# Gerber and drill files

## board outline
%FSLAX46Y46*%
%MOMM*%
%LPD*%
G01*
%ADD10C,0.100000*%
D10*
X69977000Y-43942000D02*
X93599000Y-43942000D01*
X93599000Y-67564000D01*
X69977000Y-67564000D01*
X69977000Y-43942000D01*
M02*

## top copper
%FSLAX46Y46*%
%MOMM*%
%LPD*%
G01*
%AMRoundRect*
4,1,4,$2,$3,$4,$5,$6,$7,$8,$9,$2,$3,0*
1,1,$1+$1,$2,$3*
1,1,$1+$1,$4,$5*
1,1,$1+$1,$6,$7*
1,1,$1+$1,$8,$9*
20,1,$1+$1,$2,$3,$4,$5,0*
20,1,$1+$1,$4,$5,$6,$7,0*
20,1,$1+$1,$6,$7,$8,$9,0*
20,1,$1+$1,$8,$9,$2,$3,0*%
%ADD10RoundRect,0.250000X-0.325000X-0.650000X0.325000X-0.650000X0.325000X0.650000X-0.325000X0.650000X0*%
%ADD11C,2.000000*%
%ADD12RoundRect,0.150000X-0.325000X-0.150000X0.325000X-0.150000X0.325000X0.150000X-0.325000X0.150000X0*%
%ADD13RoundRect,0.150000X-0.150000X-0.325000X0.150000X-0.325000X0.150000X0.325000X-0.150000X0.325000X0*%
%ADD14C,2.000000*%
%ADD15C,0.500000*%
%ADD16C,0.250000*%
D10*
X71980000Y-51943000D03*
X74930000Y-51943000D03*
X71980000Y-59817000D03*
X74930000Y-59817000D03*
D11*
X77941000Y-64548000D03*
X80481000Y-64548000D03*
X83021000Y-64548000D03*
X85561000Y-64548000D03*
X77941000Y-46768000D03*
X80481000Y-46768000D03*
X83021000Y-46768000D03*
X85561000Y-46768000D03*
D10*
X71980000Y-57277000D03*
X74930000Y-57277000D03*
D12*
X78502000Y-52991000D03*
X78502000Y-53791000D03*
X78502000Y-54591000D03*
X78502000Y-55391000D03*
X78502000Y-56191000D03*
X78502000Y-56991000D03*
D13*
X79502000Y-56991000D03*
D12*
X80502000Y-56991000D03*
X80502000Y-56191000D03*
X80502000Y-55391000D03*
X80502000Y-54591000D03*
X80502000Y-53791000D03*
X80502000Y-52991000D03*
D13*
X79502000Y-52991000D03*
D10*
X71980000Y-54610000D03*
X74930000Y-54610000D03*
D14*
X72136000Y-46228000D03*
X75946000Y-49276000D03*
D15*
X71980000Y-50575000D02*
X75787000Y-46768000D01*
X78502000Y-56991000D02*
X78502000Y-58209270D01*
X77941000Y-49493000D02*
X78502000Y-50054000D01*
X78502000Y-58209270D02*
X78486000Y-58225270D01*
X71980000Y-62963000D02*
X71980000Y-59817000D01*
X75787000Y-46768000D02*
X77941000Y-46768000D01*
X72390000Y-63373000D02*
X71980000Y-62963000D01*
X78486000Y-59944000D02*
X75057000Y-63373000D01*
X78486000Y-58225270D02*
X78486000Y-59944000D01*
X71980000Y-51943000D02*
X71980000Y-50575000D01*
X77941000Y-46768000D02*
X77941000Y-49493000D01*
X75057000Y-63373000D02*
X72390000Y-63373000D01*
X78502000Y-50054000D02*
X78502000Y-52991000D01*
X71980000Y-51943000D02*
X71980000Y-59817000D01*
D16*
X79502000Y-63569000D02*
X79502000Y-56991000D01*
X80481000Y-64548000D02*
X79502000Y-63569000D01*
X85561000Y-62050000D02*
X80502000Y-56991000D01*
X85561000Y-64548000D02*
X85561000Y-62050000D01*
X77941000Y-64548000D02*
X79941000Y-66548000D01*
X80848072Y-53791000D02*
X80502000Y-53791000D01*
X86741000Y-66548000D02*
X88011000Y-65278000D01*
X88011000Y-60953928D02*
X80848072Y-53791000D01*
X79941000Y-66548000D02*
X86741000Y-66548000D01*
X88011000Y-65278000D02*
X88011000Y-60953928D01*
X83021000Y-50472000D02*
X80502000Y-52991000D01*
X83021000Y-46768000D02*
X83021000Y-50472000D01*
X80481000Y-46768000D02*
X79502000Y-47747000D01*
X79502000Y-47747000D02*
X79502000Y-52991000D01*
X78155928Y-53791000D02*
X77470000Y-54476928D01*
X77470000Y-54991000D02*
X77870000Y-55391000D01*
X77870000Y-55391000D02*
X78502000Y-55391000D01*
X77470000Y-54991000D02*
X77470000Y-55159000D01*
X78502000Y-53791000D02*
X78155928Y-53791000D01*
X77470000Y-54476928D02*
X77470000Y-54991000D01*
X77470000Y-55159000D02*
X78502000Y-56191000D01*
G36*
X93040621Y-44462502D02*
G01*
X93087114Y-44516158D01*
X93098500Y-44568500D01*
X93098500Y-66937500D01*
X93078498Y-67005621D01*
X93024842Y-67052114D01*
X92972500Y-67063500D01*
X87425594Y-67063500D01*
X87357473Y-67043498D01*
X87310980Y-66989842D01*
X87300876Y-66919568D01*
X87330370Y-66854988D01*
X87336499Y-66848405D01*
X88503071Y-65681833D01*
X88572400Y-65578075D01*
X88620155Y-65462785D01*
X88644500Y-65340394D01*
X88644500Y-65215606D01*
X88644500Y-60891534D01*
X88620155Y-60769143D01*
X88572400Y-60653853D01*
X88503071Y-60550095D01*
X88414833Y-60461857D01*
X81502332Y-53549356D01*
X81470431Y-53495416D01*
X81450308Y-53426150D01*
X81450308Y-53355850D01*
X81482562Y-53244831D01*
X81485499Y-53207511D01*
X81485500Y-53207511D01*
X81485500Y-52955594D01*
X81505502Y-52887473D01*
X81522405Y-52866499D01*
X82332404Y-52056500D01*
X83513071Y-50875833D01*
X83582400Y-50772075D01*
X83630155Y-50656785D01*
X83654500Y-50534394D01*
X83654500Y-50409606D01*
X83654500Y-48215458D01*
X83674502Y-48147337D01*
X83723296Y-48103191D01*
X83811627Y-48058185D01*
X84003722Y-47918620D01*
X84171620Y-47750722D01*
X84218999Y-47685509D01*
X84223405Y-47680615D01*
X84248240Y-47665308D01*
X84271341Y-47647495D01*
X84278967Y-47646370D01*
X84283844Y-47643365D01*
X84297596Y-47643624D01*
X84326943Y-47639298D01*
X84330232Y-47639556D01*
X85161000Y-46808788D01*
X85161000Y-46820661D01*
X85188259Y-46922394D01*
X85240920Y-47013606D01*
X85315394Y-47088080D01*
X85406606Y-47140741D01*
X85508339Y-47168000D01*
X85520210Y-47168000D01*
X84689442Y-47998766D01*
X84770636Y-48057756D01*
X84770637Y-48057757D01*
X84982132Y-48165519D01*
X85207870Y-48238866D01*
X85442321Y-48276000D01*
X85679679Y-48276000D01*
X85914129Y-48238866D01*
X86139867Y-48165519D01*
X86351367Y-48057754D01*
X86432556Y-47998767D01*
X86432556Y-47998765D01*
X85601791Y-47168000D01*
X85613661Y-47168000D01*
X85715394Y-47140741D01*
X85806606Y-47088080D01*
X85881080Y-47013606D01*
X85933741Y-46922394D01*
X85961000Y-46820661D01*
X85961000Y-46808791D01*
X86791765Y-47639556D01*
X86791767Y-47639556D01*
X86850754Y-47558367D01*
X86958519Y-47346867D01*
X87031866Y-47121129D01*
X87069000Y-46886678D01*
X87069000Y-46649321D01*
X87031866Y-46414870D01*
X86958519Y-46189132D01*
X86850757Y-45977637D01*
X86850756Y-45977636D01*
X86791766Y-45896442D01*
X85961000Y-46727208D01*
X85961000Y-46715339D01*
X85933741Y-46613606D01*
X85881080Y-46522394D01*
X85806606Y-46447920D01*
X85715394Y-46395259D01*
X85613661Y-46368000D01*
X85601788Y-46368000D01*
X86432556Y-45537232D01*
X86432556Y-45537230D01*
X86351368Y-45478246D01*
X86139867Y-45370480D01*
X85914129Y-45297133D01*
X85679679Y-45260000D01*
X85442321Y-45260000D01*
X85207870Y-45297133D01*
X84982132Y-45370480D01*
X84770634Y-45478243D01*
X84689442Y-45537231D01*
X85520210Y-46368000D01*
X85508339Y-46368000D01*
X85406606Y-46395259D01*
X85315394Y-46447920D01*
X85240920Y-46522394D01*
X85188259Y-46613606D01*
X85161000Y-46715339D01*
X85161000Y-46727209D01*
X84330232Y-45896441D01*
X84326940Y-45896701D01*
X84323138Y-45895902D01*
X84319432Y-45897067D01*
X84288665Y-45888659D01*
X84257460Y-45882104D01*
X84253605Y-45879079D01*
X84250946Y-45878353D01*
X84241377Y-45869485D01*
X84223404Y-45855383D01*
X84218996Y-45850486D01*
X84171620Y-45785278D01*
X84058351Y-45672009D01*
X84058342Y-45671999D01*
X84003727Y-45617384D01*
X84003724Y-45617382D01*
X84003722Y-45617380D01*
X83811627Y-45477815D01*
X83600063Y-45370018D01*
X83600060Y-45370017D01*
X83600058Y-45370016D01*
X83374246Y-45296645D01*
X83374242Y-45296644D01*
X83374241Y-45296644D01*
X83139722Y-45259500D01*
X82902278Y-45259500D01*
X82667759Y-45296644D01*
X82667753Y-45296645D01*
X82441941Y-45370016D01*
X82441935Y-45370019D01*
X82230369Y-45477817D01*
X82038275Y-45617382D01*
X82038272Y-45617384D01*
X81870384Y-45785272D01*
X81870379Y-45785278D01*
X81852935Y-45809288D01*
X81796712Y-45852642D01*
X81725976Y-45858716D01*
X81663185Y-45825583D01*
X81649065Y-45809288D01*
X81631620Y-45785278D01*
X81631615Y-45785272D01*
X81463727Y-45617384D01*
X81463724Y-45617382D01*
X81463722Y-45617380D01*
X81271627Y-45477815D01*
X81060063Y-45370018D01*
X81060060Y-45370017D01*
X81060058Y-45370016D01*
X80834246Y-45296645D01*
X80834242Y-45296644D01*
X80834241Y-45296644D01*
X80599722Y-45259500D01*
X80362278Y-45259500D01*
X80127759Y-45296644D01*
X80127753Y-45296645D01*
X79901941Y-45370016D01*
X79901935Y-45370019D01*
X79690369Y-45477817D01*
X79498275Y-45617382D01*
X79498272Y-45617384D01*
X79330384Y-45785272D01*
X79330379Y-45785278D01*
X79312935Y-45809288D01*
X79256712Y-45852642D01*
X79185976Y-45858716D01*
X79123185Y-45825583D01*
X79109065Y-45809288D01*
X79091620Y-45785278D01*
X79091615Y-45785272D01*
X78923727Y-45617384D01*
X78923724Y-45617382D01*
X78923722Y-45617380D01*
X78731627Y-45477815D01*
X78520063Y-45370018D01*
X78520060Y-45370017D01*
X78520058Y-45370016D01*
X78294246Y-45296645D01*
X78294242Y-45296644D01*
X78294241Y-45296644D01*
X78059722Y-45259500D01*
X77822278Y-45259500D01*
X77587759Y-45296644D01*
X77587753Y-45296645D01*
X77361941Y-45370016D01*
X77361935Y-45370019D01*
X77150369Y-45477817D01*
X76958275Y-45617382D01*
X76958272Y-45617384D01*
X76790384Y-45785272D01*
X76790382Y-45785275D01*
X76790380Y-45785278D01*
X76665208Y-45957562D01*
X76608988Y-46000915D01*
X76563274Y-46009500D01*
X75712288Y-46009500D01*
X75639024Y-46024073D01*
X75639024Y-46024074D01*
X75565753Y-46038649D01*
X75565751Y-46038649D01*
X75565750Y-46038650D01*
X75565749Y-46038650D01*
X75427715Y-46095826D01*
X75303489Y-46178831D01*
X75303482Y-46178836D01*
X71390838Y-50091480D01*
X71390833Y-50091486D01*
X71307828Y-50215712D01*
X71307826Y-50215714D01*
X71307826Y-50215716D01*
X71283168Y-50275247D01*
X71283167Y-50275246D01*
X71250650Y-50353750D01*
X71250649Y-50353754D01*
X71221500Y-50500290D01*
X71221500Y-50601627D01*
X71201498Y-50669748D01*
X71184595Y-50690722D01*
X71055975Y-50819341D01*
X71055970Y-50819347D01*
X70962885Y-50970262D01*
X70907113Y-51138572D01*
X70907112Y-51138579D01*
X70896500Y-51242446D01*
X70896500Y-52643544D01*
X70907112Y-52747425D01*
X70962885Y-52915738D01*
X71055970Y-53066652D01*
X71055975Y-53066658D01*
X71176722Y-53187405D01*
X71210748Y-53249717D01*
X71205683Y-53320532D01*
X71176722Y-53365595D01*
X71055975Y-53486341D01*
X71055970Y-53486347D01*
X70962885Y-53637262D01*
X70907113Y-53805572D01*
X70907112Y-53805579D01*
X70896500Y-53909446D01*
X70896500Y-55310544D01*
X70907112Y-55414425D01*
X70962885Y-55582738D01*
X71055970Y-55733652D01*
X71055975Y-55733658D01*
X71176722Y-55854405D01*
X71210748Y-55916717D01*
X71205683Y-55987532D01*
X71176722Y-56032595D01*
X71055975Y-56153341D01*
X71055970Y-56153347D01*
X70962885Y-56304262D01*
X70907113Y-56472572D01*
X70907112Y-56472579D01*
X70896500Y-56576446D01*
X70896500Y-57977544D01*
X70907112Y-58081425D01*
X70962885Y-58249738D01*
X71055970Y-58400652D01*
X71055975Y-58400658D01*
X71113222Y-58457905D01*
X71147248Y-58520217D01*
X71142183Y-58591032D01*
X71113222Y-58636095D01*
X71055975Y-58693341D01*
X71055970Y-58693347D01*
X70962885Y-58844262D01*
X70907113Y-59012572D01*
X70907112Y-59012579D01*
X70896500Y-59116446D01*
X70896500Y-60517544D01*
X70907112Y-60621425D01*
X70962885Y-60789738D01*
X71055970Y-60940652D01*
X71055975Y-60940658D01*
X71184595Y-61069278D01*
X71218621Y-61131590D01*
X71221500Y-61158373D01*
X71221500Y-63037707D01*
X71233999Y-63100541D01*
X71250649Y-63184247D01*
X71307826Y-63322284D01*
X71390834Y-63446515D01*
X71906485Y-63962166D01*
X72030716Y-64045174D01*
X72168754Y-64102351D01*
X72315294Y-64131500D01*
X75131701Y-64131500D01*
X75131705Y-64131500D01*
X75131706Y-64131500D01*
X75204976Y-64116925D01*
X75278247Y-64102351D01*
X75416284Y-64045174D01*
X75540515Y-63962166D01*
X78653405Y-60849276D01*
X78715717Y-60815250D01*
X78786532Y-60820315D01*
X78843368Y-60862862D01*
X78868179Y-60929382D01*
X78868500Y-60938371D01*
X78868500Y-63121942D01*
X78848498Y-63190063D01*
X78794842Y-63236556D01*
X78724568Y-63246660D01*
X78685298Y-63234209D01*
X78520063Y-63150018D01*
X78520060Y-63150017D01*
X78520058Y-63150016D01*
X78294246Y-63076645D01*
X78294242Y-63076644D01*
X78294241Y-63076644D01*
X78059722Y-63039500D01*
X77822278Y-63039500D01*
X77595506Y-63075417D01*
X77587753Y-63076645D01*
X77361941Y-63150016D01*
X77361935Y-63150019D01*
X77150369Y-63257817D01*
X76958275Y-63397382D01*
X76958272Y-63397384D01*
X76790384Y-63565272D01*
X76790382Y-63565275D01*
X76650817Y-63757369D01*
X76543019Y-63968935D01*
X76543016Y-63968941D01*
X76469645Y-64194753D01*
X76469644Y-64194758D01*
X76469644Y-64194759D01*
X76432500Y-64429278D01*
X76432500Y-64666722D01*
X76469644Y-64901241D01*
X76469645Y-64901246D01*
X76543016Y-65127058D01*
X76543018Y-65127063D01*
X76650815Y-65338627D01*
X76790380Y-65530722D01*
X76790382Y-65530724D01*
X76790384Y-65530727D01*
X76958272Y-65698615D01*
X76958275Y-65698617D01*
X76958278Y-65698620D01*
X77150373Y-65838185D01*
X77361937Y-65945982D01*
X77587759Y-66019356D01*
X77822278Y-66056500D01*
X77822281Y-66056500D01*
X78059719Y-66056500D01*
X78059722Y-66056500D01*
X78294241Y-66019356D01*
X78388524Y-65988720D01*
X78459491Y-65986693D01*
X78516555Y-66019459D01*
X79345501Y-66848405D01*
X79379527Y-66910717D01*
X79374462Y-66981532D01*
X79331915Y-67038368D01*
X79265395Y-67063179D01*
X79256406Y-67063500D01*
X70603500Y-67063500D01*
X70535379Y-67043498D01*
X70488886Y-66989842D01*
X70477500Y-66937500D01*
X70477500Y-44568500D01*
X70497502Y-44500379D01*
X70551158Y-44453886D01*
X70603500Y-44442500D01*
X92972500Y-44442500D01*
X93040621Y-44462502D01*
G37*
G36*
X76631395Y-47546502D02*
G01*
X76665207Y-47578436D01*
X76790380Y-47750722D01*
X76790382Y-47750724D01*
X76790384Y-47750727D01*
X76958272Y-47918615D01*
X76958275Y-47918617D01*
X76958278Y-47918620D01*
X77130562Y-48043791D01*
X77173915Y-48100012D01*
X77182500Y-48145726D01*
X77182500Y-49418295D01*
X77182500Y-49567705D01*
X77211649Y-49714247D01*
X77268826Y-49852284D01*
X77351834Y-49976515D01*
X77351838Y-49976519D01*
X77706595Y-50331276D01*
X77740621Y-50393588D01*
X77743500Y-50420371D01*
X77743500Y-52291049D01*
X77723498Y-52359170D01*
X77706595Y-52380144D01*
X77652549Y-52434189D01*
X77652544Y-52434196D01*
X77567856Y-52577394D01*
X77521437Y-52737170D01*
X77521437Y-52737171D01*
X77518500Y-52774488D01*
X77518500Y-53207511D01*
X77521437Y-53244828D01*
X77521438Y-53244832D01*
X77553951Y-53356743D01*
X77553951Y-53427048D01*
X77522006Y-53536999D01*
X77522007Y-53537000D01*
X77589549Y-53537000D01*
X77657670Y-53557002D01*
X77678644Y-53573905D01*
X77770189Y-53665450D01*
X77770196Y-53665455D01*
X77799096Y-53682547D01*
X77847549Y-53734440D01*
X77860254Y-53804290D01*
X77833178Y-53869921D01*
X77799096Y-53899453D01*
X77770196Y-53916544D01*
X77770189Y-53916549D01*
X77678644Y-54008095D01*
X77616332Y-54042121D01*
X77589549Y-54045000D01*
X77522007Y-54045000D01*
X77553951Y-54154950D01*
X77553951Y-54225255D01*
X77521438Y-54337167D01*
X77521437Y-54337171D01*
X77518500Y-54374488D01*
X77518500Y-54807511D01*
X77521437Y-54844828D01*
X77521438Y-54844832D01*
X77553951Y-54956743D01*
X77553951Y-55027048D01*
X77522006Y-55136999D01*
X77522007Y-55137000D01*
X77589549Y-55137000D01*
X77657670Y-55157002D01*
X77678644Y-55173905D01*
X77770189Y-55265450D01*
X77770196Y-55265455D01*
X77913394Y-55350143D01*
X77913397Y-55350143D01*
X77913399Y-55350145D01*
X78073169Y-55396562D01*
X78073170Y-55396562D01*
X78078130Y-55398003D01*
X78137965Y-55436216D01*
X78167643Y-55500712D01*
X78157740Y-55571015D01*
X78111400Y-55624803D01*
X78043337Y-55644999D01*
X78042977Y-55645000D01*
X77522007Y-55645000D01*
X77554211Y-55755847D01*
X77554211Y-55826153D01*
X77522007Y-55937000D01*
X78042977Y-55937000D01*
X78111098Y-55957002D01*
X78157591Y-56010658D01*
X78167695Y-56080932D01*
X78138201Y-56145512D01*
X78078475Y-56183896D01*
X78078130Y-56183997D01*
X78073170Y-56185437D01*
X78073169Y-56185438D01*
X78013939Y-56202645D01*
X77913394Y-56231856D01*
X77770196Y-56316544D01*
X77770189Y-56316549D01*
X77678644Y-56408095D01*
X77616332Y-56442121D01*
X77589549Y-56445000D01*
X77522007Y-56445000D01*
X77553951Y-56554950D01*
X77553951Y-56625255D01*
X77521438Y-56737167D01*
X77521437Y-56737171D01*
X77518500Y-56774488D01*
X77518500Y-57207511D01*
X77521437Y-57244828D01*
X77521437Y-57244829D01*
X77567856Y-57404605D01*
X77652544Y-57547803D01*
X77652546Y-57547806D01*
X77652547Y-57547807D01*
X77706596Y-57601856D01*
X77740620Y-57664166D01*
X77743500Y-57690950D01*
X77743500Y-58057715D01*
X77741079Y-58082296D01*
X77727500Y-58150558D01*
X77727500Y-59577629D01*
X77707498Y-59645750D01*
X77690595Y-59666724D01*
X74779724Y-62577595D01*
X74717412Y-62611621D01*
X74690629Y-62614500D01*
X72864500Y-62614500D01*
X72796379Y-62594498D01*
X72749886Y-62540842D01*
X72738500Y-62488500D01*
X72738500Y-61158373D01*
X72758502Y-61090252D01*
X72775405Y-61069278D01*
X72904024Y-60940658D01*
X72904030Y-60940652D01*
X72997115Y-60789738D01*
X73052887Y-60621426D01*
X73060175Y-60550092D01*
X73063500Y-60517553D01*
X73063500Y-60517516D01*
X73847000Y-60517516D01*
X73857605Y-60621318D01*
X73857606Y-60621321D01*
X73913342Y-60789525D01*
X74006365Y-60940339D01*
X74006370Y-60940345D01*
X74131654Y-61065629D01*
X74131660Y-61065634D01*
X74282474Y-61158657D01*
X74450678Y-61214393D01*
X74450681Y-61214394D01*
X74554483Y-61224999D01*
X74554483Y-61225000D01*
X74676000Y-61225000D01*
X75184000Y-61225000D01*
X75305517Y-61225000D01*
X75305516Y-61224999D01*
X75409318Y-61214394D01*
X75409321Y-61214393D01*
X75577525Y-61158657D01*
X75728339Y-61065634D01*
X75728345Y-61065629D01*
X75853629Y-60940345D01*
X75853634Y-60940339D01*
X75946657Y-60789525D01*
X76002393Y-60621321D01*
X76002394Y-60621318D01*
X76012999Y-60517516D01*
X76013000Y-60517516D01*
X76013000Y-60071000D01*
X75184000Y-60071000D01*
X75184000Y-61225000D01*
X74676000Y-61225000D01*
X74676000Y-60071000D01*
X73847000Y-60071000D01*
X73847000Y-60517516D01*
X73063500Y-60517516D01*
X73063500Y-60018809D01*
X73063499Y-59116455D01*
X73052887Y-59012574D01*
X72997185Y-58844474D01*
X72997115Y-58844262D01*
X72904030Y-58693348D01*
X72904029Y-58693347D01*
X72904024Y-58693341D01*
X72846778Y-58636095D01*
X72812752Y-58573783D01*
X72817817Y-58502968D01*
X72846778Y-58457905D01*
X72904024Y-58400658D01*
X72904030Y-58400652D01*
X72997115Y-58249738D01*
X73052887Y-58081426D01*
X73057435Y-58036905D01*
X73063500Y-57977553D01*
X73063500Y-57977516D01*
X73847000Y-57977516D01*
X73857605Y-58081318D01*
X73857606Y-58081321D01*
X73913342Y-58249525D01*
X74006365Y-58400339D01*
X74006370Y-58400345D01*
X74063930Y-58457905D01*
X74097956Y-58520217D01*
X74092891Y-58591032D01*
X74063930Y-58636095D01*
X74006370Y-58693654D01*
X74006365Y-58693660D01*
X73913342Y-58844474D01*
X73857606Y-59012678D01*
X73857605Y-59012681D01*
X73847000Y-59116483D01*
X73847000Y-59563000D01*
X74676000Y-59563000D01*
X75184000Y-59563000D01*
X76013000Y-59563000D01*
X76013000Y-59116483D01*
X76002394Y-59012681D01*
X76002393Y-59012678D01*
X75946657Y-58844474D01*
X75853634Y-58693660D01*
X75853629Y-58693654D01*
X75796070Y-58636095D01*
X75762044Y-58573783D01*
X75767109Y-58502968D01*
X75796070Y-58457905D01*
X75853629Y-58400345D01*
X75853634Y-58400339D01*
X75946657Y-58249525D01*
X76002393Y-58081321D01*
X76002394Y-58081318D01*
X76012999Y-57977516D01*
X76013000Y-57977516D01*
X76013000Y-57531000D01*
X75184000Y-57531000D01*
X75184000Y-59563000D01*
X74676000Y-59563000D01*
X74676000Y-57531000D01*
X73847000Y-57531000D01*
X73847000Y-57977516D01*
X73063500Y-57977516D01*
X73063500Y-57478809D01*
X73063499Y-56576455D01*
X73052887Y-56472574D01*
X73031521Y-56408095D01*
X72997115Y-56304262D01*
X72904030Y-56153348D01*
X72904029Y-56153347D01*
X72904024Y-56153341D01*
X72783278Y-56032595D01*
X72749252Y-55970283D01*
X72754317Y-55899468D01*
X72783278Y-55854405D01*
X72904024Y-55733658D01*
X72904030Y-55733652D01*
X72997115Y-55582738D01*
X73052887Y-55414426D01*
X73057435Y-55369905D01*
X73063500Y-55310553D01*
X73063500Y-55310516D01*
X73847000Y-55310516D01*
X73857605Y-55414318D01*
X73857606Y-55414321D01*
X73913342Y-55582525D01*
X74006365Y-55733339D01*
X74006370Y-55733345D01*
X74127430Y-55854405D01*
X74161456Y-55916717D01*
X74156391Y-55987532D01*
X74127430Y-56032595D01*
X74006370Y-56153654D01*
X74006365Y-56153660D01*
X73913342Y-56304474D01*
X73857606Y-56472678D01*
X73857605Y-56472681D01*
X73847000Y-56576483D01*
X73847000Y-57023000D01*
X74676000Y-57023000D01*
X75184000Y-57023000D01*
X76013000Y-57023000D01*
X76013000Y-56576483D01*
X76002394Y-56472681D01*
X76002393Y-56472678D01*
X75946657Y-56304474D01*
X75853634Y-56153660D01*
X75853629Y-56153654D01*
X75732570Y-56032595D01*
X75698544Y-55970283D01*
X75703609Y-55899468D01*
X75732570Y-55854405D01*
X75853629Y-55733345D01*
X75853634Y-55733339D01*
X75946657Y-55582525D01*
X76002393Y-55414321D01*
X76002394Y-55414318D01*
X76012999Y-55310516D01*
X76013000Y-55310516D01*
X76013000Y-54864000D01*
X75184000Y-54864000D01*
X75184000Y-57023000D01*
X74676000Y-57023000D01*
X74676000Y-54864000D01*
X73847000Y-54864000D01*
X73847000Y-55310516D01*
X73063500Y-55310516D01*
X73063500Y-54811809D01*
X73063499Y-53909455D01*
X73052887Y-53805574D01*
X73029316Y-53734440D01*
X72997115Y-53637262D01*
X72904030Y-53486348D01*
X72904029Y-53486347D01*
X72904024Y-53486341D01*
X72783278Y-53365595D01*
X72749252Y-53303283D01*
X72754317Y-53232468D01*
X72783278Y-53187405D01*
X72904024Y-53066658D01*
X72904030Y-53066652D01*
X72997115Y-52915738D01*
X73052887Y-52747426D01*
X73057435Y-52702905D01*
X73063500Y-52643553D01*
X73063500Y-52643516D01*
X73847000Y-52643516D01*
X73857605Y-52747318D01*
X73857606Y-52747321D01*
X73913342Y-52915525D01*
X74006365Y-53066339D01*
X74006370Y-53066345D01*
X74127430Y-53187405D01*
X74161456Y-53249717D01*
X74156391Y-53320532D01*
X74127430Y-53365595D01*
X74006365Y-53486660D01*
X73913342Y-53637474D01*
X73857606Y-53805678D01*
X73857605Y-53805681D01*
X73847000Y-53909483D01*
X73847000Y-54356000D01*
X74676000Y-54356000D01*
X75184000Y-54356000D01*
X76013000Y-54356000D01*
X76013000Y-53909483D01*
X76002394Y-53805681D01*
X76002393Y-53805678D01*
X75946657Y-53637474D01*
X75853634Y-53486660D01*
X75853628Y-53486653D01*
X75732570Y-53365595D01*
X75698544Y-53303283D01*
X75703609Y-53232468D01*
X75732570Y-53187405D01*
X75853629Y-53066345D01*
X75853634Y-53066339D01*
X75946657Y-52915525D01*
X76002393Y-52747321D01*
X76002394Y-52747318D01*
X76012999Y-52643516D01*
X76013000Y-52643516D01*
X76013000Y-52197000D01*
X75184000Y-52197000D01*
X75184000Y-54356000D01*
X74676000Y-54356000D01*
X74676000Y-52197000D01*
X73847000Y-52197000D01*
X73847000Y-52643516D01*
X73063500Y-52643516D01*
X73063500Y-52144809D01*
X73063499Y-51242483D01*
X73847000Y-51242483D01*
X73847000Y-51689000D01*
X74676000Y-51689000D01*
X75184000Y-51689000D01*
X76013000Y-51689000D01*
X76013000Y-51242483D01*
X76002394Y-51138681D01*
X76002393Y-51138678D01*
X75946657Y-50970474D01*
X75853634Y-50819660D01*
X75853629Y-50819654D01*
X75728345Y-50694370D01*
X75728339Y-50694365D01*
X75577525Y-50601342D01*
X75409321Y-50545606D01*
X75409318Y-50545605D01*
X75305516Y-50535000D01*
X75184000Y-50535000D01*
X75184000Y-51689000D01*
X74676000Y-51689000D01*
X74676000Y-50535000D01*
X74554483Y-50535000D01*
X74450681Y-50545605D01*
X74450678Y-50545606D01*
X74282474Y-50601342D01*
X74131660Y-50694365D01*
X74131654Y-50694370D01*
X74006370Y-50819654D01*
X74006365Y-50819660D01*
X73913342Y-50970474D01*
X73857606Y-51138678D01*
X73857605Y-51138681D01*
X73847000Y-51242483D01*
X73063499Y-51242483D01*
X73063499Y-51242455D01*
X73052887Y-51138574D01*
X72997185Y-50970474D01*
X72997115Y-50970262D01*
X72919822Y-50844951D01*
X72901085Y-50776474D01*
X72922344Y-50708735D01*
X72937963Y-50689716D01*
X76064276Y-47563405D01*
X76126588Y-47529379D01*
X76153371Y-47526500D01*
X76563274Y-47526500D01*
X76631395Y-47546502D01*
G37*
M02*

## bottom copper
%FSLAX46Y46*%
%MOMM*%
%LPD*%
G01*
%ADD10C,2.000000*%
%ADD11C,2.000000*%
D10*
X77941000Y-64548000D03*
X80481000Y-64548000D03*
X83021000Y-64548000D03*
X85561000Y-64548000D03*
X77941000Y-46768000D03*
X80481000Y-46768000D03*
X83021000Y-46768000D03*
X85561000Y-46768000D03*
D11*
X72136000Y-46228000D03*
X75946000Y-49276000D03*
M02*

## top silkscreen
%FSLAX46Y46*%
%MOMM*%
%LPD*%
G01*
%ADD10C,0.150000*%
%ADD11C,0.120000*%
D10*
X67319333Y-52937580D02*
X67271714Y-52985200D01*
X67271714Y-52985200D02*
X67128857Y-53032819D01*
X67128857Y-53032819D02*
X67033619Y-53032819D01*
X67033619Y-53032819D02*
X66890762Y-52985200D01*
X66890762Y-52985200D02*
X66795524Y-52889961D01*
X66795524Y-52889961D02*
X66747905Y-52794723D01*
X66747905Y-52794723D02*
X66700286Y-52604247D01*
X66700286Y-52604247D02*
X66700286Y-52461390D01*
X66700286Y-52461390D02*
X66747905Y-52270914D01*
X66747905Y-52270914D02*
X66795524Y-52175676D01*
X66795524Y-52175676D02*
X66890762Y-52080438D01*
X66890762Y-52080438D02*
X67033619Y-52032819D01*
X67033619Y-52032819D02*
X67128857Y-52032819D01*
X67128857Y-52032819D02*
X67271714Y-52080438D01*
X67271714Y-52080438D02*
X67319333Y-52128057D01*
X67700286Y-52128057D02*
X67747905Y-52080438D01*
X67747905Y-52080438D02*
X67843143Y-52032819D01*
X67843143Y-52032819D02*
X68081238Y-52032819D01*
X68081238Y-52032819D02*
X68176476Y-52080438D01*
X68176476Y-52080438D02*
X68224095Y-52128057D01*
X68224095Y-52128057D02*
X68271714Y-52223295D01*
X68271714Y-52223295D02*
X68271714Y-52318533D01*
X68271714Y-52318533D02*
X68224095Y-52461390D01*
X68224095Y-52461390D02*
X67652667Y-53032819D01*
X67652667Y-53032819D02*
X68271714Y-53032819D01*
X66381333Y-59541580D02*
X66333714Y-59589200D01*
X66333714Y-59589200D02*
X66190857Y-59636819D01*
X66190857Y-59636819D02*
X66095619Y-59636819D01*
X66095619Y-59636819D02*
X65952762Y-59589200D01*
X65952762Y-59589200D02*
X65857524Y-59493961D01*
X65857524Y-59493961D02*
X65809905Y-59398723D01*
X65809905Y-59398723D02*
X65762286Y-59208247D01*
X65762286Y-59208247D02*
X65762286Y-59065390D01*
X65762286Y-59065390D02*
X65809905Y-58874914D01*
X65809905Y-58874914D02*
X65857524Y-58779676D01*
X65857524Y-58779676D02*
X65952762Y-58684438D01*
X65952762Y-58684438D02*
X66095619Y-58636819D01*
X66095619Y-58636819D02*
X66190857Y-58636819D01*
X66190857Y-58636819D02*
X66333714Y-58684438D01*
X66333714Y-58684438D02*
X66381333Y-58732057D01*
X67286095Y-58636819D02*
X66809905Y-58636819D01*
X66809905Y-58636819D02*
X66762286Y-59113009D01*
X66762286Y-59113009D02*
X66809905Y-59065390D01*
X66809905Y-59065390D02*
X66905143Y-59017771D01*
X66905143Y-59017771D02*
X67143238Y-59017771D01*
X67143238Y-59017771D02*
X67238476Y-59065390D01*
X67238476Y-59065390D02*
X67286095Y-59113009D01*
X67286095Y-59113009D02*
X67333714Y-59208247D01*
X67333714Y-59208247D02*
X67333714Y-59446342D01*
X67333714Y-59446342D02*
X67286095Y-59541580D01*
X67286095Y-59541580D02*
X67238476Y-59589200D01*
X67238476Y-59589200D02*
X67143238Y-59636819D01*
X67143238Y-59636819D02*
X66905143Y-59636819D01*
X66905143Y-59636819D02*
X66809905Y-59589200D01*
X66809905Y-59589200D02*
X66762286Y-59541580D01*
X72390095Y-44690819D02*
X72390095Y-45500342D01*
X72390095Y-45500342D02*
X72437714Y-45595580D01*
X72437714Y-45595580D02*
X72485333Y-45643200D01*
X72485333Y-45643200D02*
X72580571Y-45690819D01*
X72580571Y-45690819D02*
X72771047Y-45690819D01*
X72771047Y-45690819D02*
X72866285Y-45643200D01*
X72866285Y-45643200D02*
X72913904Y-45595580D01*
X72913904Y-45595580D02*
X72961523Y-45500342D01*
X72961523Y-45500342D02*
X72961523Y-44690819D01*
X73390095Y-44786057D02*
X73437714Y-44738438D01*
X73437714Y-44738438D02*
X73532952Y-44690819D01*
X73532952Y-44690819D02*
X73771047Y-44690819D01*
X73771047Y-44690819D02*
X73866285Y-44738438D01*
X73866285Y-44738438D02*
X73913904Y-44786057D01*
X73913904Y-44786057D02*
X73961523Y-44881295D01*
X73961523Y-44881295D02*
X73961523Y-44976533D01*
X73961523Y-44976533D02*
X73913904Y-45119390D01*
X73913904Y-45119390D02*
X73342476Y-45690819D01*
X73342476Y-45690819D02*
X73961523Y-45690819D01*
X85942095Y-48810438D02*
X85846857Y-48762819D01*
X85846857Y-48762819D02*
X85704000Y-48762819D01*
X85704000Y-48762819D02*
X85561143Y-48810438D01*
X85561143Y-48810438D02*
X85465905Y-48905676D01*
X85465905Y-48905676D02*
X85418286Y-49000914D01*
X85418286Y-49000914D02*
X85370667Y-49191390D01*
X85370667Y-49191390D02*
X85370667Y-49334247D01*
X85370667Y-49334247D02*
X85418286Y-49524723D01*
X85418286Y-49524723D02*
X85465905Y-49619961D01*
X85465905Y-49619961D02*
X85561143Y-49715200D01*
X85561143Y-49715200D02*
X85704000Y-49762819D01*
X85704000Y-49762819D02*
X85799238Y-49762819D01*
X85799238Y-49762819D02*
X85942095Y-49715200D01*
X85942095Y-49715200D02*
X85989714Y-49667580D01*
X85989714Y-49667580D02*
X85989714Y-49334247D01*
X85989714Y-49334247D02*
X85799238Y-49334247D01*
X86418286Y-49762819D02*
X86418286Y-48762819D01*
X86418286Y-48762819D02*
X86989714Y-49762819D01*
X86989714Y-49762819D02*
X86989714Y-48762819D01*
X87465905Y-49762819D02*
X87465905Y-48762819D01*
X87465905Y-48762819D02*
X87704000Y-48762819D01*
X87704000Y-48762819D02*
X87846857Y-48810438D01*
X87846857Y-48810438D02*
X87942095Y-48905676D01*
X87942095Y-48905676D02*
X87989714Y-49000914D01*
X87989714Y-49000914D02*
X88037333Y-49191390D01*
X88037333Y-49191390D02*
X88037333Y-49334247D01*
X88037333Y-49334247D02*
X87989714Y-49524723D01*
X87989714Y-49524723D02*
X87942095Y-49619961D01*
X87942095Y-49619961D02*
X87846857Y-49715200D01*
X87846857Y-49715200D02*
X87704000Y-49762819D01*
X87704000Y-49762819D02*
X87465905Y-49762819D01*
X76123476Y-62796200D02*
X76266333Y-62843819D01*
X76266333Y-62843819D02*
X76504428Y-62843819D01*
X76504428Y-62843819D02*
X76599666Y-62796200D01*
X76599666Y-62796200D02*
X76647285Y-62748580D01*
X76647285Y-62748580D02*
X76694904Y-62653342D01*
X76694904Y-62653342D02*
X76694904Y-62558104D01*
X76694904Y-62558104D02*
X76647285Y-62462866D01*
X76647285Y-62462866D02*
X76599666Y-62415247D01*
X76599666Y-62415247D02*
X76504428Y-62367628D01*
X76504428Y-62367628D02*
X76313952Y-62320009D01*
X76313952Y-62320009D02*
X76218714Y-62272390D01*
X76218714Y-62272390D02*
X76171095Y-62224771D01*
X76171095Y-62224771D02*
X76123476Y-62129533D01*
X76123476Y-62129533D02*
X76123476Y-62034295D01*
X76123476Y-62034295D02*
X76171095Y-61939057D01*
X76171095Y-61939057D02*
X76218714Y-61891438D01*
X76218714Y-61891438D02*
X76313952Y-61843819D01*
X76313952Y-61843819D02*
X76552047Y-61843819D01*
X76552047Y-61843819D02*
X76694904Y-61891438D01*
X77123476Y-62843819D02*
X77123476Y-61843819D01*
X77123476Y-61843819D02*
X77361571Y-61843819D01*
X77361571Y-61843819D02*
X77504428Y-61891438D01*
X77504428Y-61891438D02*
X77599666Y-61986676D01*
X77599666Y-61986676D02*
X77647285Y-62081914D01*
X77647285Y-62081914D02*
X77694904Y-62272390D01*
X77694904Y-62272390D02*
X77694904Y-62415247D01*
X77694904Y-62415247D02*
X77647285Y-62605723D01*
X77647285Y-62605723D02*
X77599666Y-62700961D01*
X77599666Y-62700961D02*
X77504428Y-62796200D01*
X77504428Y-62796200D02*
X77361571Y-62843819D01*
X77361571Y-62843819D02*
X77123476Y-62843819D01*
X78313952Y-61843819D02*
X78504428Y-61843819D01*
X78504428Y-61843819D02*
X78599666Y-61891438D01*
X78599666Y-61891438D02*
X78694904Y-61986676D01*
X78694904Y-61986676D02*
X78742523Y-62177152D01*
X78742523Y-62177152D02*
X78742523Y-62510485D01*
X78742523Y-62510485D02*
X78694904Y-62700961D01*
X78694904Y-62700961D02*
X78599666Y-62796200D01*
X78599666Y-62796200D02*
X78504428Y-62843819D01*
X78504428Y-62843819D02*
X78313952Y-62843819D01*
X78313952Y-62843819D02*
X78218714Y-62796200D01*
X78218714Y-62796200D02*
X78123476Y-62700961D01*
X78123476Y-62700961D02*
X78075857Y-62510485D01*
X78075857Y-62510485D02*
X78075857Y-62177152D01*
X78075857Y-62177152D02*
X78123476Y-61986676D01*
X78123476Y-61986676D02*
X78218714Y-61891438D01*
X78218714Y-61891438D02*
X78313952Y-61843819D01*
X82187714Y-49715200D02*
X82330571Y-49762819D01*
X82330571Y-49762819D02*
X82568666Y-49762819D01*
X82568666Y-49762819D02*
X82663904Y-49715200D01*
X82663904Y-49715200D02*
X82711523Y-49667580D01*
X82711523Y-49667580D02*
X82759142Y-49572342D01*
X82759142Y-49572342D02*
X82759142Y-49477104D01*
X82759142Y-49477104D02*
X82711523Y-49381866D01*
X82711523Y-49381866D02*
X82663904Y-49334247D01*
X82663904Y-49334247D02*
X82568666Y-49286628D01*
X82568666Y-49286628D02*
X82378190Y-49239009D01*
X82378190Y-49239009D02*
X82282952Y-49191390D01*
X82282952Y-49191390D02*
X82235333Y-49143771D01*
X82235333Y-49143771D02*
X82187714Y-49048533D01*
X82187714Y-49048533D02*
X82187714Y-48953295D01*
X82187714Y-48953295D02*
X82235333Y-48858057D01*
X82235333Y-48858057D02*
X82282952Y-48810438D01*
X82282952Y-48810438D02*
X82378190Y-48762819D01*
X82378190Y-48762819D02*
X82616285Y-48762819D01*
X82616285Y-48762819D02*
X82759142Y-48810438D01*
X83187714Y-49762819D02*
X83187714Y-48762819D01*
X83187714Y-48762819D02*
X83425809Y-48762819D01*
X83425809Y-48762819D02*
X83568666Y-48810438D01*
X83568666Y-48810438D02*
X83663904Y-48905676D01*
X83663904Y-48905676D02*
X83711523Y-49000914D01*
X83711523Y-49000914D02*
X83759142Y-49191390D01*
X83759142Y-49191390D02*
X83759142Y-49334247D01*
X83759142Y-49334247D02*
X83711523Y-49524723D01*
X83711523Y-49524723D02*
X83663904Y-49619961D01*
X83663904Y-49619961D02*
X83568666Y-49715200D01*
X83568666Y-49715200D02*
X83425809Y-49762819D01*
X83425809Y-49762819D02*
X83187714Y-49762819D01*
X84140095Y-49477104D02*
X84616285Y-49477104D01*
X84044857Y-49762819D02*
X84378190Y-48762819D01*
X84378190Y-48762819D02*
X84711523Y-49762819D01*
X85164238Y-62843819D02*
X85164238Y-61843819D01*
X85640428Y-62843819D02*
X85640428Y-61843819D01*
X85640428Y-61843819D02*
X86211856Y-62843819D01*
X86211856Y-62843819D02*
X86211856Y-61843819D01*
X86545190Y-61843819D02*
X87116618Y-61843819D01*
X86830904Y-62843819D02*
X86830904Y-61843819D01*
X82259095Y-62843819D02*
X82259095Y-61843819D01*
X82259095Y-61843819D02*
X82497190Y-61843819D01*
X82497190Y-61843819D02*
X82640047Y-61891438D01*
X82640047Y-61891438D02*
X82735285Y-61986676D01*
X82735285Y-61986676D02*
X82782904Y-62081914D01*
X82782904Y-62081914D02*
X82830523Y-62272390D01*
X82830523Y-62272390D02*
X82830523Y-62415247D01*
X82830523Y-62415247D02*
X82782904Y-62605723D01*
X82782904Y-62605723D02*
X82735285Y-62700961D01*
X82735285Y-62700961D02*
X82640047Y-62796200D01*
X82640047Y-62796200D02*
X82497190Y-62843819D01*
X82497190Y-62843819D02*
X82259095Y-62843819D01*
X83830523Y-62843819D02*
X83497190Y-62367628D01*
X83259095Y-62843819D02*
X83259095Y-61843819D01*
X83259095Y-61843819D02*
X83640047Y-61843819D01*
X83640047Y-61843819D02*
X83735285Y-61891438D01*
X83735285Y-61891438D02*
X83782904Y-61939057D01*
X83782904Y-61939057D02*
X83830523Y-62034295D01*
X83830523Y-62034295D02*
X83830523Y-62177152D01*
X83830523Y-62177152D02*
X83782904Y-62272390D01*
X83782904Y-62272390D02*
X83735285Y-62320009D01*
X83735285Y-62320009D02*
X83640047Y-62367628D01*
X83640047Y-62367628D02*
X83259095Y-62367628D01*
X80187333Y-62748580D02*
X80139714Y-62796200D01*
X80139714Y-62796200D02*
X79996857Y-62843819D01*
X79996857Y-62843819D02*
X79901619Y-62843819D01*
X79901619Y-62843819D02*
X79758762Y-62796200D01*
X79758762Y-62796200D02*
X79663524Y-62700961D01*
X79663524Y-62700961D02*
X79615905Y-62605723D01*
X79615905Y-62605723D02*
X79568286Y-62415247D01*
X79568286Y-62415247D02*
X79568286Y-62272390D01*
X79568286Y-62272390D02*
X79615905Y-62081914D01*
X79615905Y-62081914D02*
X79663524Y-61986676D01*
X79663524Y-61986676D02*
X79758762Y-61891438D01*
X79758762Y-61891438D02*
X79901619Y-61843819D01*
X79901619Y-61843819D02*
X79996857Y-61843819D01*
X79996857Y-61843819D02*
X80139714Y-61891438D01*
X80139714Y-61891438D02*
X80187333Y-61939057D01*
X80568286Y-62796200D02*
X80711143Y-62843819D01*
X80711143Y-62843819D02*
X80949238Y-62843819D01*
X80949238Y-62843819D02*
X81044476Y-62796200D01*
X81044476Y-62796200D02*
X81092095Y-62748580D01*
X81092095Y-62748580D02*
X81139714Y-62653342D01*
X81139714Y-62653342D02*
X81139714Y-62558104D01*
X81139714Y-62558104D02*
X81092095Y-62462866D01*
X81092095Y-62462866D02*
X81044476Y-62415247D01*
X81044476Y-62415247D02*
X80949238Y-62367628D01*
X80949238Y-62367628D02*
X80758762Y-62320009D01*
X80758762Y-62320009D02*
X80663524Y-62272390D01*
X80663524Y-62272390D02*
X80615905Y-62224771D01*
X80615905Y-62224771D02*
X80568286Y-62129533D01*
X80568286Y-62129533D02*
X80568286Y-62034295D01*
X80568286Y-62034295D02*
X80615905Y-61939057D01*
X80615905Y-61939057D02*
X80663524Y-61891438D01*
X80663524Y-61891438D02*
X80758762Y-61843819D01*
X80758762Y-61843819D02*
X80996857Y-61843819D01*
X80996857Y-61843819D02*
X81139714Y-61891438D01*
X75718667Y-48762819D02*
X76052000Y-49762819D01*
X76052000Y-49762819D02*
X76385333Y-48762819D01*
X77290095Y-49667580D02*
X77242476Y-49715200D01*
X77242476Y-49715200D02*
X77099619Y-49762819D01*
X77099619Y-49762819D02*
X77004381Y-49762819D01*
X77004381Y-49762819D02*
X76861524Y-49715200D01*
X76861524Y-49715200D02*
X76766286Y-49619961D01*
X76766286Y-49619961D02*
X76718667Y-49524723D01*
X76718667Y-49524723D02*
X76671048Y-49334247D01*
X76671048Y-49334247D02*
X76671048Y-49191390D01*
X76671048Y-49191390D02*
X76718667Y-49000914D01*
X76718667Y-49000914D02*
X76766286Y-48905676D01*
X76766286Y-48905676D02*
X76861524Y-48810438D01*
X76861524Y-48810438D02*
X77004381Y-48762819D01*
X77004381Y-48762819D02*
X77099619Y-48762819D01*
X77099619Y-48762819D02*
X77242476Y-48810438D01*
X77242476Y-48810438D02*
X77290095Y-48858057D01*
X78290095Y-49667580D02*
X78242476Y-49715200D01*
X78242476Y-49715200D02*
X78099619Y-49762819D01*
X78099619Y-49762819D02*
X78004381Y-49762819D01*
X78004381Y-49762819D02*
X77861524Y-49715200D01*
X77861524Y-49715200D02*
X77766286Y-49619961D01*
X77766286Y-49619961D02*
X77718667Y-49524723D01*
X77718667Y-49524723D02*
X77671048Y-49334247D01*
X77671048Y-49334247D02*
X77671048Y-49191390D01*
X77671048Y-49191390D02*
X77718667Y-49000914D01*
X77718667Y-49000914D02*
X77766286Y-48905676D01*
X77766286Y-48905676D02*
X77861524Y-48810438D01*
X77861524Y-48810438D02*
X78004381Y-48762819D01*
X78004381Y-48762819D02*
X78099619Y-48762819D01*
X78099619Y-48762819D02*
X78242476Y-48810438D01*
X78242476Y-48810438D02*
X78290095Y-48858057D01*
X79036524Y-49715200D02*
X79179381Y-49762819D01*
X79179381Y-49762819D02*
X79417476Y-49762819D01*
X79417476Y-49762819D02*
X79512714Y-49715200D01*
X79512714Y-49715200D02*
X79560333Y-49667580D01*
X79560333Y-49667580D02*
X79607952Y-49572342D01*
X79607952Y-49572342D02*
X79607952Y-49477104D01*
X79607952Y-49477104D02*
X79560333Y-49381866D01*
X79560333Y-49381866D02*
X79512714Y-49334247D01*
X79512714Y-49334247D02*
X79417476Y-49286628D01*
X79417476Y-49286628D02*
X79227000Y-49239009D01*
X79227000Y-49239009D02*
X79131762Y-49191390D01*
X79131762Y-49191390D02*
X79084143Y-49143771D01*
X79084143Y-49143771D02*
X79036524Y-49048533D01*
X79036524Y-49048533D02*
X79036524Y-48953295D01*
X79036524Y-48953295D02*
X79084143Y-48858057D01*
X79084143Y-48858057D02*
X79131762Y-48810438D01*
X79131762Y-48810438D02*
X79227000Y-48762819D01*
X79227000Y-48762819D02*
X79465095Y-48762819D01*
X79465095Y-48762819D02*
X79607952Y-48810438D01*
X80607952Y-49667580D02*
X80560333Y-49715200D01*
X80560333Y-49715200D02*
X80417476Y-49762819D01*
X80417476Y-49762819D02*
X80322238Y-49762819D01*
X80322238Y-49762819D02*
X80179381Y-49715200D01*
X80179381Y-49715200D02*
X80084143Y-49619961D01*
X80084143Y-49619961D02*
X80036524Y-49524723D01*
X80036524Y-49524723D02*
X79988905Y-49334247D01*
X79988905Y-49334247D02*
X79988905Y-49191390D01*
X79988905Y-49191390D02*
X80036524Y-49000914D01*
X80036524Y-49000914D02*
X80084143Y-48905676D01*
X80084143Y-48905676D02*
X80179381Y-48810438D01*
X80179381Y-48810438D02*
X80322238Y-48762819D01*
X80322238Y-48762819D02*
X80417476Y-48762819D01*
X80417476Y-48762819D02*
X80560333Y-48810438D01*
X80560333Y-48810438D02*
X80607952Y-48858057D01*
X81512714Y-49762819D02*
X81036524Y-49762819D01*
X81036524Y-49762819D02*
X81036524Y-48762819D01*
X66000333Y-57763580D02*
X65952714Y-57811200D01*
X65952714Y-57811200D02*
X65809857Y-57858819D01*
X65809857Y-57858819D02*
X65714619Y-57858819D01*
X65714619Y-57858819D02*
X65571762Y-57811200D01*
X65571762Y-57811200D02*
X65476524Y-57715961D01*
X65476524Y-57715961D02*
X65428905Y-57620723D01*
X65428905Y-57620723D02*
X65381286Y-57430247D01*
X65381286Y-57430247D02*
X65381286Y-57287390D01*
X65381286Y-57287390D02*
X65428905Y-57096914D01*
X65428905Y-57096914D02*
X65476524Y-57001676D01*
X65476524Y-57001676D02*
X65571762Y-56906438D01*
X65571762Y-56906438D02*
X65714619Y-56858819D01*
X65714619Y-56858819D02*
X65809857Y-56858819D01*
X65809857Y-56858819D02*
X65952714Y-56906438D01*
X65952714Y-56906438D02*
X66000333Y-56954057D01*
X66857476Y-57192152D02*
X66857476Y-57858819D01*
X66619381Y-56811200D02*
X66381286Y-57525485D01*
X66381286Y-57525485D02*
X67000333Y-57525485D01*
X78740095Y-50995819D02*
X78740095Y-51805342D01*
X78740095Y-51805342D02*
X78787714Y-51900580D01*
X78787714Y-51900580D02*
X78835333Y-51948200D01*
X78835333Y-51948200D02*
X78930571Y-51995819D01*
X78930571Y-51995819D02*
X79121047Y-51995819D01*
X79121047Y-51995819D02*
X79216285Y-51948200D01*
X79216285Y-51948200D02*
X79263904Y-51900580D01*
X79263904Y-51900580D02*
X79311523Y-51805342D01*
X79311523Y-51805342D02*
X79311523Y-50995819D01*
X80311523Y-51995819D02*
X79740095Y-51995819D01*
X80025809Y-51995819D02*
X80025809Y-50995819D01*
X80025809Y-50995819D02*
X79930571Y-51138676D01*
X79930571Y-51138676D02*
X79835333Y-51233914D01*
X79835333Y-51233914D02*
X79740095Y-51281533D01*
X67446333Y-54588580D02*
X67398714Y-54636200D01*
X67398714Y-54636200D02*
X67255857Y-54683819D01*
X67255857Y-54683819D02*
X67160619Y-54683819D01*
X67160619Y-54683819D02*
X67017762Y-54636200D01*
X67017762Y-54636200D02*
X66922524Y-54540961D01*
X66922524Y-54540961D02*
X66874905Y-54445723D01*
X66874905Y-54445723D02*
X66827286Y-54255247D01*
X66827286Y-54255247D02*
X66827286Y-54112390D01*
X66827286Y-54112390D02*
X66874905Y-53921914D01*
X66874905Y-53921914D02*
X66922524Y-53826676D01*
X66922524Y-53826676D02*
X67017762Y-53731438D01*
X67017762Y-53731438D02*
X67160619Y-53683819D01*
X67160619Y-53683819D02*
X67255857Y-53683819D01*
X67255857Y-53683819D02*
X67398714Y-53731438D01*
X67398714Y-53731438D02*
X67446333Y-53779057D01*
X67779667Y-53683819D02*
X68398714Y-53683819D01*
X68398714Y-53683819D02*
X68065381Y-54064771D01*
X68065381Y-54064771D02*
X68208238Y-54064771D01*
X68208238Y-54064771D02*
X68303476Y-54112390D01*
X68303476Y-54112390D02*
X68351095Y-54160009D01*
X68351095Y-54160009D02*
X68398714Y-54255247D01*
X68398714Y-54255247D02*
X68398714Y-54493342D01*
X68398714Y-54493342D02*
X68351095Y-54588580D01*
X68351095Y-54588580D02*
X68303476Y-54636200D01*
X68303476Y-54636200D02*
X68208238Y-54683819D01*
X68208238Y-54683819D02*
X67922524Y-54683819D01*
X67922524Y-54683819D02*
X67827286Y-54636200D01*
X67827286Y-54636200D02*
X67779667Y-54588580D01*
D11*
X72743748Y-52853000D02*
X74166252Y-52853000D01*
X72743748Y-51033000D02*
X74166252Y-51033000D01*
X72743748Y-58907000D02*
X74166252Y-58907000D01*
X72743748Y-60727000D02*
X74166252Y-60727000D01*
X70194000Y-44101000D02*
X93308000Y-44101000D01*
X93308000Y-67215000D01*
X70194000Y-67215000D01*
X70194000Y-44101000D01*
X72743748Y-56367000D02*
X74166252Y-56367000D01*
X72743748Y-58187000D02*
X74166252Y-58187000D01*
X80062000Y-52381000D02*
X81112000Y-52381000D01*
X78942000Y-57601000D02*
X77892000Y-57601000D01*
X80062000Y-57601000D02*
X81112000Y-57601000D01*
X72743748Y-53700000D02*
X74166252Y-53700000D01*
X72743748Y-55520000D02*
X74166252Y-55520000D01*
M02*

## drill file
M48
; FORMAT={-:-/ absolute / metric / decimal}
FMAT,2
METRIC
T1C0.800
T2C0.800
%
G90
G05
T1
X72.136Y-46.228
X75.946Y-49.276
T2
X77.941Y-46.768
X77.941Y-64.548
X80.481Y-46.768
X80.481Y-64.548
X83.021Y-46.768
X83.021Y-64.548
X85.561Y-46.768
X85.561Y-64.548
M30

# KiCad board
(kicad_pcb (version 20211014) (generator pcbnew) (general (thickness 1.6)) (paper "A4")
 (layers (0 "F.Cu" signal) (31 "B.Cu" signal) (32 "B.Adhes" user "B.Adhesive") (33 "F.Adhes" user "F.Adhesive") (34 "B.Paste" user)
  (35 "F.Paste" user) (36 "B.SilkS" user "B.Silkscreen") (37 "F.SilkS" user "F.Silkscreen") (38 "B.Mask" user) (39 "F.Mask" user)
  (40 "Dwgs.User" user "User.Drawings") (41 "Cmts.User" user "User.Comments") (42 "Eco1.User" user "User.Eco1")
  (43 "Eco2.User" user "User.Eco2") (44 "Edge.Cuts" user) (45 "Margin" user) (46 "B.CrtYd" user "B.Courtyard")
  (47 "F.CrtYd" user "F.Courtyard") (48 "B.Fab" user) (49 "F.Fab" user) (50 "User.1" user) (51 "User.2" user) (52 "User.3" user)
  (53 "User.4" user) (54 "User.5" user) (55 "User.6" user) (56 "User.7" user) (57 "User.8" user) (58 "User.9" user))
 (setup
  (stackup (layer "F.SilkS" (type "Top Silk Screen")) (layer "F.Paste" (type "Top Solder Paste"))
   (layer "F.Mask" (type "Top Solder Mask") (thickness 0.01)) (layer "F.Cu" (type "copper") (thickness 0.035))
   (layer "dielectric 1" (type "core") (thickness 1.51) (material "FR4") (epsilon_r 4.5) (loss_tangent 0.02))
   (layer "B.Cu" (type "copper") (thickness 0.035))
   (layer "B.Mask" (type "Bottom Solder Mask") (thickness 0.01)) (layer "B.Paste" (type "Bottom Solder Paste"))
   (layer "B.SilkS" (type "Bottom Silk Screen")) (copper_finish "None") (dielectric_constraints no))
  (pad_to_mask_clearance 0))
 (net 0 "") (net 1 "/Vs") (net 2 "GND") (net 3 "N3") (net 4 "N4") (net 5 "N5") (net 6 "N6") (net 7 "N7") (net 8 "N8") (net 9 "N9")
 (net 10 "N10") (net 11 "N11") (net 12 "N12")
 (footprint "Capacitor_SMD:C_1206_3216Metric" (layer "F.Cu") (at 73.455 51.943)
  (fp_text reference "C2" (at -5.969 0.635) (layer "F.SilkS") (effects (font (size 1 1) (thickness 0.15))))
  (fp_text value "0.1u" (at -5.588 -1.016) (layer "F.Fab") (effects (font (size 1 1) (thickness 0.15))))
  (fp_line (start -0.711252 0.91) (end 0.711252 0.91) (layer "F.SilkS") (width 0.12))
  (fp_line (start -0.711252 -0.91) (end 0.711252 -0.91) (layer "F.SilkS") (width 0.12))
  (pad "1" smd roundrect (at -1.475 0) (size 1.15 1.8) (layers "F.Cu" "F.Paste" "F.Mask") (roundrect_rratio 0.2173913043) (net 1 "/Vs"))
  (pad "2" smd roundrect (at 1.475 0) (size 1.15 1.8) (layers "F.Cu" "F.Paste" "F.Mask") (roundrect_rratio 0.2173913043) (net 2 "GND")))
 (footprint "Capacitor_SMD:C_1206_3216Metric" (layer "F.Cu") (at 73.455 59.817)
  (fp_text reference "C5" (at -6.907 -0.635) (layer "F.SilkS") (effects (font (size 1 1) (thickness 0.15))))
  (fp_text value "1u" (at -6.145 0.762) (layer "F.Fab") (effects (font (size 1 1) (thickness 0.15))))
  (fp_line (start -0.711252 -0.91) (end 0.711252 -0.91) (layer "F.SilkS") (width 0.12))
  (fp_line (start -0.711252 0.91) (end 0.711252 0.91) (layer "F.SilkS") (width 0.12))
  (pad "1" smd roundrect (at -1.475 0) (size 1.15 1.8) (layers "F.Cu" "F.Paste" "F.Mask") (roundrect_rratio 0.2173913043) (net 1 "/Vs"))
  (pad "2" smd roundrect (at 1.475 0) (size 1.15 1.8) (layers "F.Cu" "F.Paste" "F.Mask") (roundrect_rratio 0.2173913043) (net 2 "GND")))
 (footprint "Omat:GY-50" (layer "F.Cu") (at 70.194 67.215)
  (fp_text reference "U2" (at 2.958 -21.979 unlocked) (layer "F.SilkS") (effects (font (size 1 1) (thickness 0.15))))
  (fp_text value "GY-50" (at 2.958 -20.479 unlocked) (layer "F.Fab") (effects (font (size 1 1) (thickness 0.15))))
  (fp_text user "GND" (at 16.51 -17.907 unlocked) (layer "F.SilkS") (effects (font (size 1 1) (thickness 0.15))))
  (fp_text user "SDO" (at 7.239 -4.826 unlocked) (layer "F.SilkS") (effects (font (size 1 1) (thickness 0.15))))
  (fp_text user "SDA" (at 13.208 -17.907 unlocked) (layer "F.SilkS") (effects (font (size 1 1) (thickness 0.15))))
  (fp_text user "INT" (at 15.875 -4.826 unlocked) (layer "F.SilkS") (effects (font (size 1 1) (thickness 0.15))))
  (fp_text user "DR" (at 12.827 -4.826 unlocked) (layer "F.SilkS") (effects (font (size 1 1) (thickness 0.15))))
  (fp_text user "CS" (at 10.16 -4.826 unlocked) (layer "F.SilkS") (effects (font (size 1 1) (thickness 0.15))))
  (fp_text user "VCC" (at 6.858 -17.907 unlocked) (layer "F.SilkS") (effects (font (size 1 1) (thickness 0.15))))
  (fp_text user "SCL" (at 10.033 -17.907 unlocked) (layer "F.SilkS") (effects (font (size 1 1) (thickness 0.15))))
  (fp_rect (start 0 0) (end 23.114 -23.114) (layer "F.SilkS") (width 0.12) (fill none))
  (pad "1" thru_hole circle (at 7.747 -2.667) (size 2 2) (drill 0.8) (layers *.Cu *.Mask) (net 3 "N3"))
  (pad "2" thru_hole circle (at 10.287 -2.667) (size 2 2) (drill 0.8) (layers *.Cu *.Mask) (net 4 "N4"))
  (pad "3" thru_hole circle (at 12.827 -2.667) (size 2 2) (drill 0.8) (layers *.Cu *.Mask) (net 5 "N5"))
  (pad "4" thru_hole circle (at 15.367 -2.667) (size 2 2) (drill 0.8) (layers *.Cu *.Mask) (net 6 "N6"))
  (pad "5" thru_hole circle (at 7.747 -20.447) (size 2 2) (drill 0.8) (layers *.Cu *.Mask) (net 1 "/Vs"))
  (pad "6" thru_hole circle (at 10.287 -20.447) (size 2 2) (drill 0.8) (layers *.Cu *.Mask) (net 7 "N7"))
  (pad "7" thru_hole circle (at 12.827 -20.447) (size 2 2) (drill 0.8) (layers *.Cu *.Mask) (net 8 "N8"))
  (pad "8" thru_hole circle (at 15.367 -20.447) (size 2 2) (drill 0.8) (layers *.Cu *.Mask) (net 2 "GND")))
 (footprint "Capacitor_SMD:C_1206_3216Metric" (layer "F.Cu") (at 73.455 57.277)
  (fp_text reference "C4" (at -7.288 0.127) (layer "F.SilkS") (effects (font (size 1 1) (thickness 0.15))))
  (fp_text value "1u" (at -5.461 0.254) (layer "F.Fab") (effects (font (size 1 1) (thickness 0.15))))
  (fp_line (start -0.711252 -0.91) (end 0.711252 -0.91) (layer "F.SilkS") (width 0.12))
  (fp_line (start -0.711252 0.91) (end 0.711252 0.91) (layer "F.SilkS") (width 0.12))
  (pad "1" smd roundrect (at -1.475 0) (size 1.15 1.8) (layers "F.Cu" "F.Paste" "F.Mask") (roundrect_rratio 0.2173913043) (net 1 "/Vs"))
  (pad "2" smd roundrect (at 1.475 0) (size 1.15 1.8) (layers "F.Cu" "F.Paste" "F.Mask") (roundrect_rratio 0.2173913043) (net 2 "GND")))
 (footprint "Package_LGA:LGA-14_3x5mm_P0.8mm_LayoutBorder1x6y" (layer "F.Cu") (at 79.502 54.991)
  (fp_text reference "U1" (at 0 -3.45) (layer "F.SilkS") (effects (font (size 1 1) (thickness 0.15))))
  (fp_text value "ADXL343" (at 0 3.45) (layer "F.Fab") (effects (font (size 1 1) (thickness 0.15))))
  (fp_line (start 0.56 -2.61) (end 1.61 -2.61) (layer "F.SilkS") (width 0.12))
  (fp_line (start -0.56 2.61) (end -1.61 2.61) (layer "F.SilkS") (width 0.12))
  (fp_line (start 0.56 2.61) (end 1.61 2.61) (layer "F.SilkS") (width 0.12))
  (pad "1" smd roundrect (at -1 -2) (size 0.95 0.6) (layers "F.Cu" "F.Paste" "F.Mask") (roundrect_rratio 0.25) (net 1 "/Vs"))
  (pad "2" smd roundrect (at -1 -1.2) (size 0.95 0.6) (layers "F.Cu" "F.Paste" "F.Mask") (roundrect_rratio 0.25) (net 2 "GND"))
  (pad "3" smd roundrect (at -1 -0.4) (size 0.95 0.6) (layers "F.Cu" "F.Paste" "F.Mask") (roundrect_rratio 0.25) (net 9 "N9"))
  (pad "4" smd roundrect (at -1 0.4) (size 0.95 0.6) (layers "F.Cu" "F.Paste" "F.Mask") (roundrect_rratio 0.25) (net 2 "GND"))
  (pad "5" smd roundrect (at -1 1.2) (size 0.95 0.6) (layers "F.Cu" "F.Paste" "F.Mask") (roundrect_rratio 0.25) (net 2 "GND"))
  (pad "6" smd roundrect (at -1 2) (size 0.95 0.6) (layers "F.Cu" "F.Paste" "F.Mask") (roundrect_rratio 0.25) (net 1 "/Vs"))
  (pad "7" smd roundrect (at 0 2) (size 0.6 0.95) (layers "F.Cu" "F.Paste" "F.Mask") (roundrect_rratio 0.25) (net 4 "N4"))
  (pad "8" smd roundrect (at 1 2) (size 0.95 0.6) (layers "F.Cu" "F.Paste" "F.Mask") (roundrect_rratio 0.25) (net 6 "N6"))
  (pad "9" smd roundrect (at 1 1.2) (size 0.95 0.6) (layers "F.Cu" "F.Paste" "F.Mask") (roundrect_rratio 0.25) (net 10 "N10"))
  (pad "10" smd roundrect (at 1 0.4) (size 0.95 0.6) (layers "F.Cu" "F.Paste" "F.Mask") (roundrect_rratio 0.25) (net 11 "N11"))
  (pad "11" smd roundrect (at 1 -0.4) (size 0.95 0.6) (layers "F.Cu" "F.Paste" "F.Mask") (roundrect_rratio 0.25) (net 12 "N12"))
  (pad "12" smd roundrect (at 1 -1.2) (size 0.95 0.6) (layers "F.Cu" "F.Paste" "F.Mask") (roundrect_rratio 0.25) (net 3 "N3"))
  (pad "13" smd roundrect (at 1 -2) (size 0.95 0.6) (layers "F.Cu" "F.Paste" "F.Mask") (roundrect_rratio 0.25) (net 8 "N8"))
  (pad "14" smd roundrect (at 0 -2) (size 0.6 0.95) (layers "F.Cu" "F.Paste" "F.Mask") (roundrect_rratio 0.25) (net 7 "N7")))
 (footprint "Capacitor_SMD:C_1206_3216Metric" (layer "F.Cu") (at 73.455 54.61)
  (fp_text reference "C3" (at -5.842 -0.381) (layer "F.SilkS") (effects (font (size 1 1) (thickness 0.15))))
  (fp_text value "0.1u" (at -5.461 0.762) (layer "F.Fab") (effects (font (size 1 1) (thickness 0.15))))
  (fp_line (start -0.711252 -0.91) (end 0.711252 -0.91) (layer "F.SilkS") (width 0.12))
  (fp_line (start -0.711252 0.91) (end 0.711252 0.91) (layer "F.SilkS") (width 0.12))
  (pad "1" smd roundrect (at -1.475 0) (size 1.15 1.8) (layers "F.Cu" "F.Paste" "F.Mask") (roundrect_rratio 0.2173913043) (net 1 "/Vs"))
  (pad "2" smd roundrect (at 1.475 0) (size 1.15 1.8) (layers "F.Cu" "F.Paste" "F.Mask") (roundrect_rratio 0.2173913043) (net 2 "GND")))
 (gr_rect (start 69.977 43.942) (end 93.599 67.564) (layer "Edge.Cuts") (width 0.1) (fill none))
 (segment (start 71.98 50.575) (end 75.787 46.768) (width 0.5) (layer "F.Cu") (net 1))
 (segment (start 78.502 56.991) (end 78.502 58.20927) (width 0.5) (layer "F.Cu") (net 1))
 (segment (start 77.941 49.493) (end 78.502 50.054) (width 0.5) (layer "F.Cu") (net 1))
 (segment (start 78.502 58.20927) (end 78.486 58.22527) (width 0.5) (layer "F.Cu") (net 1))
 (segment (start 71.98 62.963) (end 71.98 59.817) (width 0.5) (layer "F.Cu") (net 1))
 (segment (start 75.787 46.768) (end 77.941 46.768) (width 0.5) (layer "F.Cu") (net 1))
 (segment (start 72.39 63.373) (end 71.98 62.963) (width 0.5) (layer "F.Cu") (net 1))
 (segment (start 78.486 59.944) (end 75.057 63.373) (width 0.5) (layer "F.Cu") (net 1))
 (segment (start 78.486 58.22527) (end 78.486 59.944) (width 0.5) (layer "F.Cu") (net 1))
 (segment (start 71.98 51.943) (end 71.98 50.575) (width 0.5) (layer "F.Cu") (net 1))
 (segment (start 77.941 46.768) (end 77.941 49.493) (width 0.5) (layer "F.Cu") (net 1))
 (segment (start 75.057 63.373) (end 72.39 63.373) (width 0.5) (layer "F.Cu") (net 1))
 (segment (start 78.502 50.054) (end 78.502 52.991) (width 0.5) (layer "F.Cu") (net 1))
 (segment (start 71.98 51.943) (end 71.98 59.817) (width 0.5) (layer "F.Cu") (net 1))
 (segment (start 79.502 63.569) (end 79.502 56.991) (width 0.25) (layer "F.Cu") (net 4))
 (segment (start 80.481 64.548) (end 79.502 63.569) (width 0.25) (layer "F.Cu") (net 4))
 (segment (start 85.561 62.05) (end 80.502 56.991) (width 0.25) (layer "F.Cu") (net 6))
 (segment (start 85.561 64.548) (end 85.561 62.05) (width 0.25) (layer "F.Cu") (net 6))
 (segment (start 77.941 64.548) (end 79.941 66.548) (width 0.25) (layer "F.Cu") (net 3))
 (segment (start 80.848072 53.791) (end 80.502 53.791) (width 0.25) (layer "F.Cu") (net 3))
 (segment (start 86.741 66.548) (end 88.011 65.278) (width 0.25) (layer "F.Cu") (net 3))
 (segment (start 88.011 60.953928) (end 80.848072 53.791) (width 0.25) (layer "F.Cu") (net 3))
 (segment (start 79.941 66.548) (end 86.741 66.548) (width 0.25) (layer "F.Cu") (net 3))
 (segment (start 88.011 65.278) (end 88.011 60.953928) (width 0.25) (layer "F.Cu") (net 3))
 (segment (start 83.021 50.472) (end 80.502 52.991) (width 0.25) (layer "F.Cu") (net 8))
 (segment (start 83.021 46.768) (end 83.021 50.472) (width 0.25) (layer "F.Cu") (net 8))
 (segment (start 80.481 46.768) (end 79.502 47.747) (width 0.25) (layer "F.Cu") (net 7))
 (segment (start 79.502 47.747) (end 79.502 52.991) (width 0.25) (layer "F.Cu") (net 7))
 (segment (start 78.155928 53.791) (end 77.47 54.476928) (width 0.25) (layer "F.Cu") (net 2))
 (segment (start 77.47 54.991) (end 77.87 55.391) (width 0.25) (layer "F.Cu") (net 2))
 (segment (start 77.87 55.391) (end 78.502 55.391) (width 0.25) (layer "F.Cu") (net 2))
 (segment (start 77.47 54.991) (end 77.47 55.159) (width 0.25) (layer "F.Cu") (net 2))
 (segment (start 78.502 53.791) (end 78.155928 53.791) (width 0.25) (layer "F.Cu") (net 2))
 (segment (start 77.47 54.476928) (end 77.47 54.991) (width 0.25) (layer "F.Cu") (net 2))
 (segment (start 77.47 55.159) (end 78.502 56.191) (width 0.25) (layer "F.Cu") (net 2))
 (via (at 72.136 46.228) (size 2) (drill 0.8) (layers "F.Cu" "B.Cu") (free) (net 2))
 (via (at 75.946 49.276) (size 2) (drill 0.8) (layers "F.Cu" "B.Cu") (free) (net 2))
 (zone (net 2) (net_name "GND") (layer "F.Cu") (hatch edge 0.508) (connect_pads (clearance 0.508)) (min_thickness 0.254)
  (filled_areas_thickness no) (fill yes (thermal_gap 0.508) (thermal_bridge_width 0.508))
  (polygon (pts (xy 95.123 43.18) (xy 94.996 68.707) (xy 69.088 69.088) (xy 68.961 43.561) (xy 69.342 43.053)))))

